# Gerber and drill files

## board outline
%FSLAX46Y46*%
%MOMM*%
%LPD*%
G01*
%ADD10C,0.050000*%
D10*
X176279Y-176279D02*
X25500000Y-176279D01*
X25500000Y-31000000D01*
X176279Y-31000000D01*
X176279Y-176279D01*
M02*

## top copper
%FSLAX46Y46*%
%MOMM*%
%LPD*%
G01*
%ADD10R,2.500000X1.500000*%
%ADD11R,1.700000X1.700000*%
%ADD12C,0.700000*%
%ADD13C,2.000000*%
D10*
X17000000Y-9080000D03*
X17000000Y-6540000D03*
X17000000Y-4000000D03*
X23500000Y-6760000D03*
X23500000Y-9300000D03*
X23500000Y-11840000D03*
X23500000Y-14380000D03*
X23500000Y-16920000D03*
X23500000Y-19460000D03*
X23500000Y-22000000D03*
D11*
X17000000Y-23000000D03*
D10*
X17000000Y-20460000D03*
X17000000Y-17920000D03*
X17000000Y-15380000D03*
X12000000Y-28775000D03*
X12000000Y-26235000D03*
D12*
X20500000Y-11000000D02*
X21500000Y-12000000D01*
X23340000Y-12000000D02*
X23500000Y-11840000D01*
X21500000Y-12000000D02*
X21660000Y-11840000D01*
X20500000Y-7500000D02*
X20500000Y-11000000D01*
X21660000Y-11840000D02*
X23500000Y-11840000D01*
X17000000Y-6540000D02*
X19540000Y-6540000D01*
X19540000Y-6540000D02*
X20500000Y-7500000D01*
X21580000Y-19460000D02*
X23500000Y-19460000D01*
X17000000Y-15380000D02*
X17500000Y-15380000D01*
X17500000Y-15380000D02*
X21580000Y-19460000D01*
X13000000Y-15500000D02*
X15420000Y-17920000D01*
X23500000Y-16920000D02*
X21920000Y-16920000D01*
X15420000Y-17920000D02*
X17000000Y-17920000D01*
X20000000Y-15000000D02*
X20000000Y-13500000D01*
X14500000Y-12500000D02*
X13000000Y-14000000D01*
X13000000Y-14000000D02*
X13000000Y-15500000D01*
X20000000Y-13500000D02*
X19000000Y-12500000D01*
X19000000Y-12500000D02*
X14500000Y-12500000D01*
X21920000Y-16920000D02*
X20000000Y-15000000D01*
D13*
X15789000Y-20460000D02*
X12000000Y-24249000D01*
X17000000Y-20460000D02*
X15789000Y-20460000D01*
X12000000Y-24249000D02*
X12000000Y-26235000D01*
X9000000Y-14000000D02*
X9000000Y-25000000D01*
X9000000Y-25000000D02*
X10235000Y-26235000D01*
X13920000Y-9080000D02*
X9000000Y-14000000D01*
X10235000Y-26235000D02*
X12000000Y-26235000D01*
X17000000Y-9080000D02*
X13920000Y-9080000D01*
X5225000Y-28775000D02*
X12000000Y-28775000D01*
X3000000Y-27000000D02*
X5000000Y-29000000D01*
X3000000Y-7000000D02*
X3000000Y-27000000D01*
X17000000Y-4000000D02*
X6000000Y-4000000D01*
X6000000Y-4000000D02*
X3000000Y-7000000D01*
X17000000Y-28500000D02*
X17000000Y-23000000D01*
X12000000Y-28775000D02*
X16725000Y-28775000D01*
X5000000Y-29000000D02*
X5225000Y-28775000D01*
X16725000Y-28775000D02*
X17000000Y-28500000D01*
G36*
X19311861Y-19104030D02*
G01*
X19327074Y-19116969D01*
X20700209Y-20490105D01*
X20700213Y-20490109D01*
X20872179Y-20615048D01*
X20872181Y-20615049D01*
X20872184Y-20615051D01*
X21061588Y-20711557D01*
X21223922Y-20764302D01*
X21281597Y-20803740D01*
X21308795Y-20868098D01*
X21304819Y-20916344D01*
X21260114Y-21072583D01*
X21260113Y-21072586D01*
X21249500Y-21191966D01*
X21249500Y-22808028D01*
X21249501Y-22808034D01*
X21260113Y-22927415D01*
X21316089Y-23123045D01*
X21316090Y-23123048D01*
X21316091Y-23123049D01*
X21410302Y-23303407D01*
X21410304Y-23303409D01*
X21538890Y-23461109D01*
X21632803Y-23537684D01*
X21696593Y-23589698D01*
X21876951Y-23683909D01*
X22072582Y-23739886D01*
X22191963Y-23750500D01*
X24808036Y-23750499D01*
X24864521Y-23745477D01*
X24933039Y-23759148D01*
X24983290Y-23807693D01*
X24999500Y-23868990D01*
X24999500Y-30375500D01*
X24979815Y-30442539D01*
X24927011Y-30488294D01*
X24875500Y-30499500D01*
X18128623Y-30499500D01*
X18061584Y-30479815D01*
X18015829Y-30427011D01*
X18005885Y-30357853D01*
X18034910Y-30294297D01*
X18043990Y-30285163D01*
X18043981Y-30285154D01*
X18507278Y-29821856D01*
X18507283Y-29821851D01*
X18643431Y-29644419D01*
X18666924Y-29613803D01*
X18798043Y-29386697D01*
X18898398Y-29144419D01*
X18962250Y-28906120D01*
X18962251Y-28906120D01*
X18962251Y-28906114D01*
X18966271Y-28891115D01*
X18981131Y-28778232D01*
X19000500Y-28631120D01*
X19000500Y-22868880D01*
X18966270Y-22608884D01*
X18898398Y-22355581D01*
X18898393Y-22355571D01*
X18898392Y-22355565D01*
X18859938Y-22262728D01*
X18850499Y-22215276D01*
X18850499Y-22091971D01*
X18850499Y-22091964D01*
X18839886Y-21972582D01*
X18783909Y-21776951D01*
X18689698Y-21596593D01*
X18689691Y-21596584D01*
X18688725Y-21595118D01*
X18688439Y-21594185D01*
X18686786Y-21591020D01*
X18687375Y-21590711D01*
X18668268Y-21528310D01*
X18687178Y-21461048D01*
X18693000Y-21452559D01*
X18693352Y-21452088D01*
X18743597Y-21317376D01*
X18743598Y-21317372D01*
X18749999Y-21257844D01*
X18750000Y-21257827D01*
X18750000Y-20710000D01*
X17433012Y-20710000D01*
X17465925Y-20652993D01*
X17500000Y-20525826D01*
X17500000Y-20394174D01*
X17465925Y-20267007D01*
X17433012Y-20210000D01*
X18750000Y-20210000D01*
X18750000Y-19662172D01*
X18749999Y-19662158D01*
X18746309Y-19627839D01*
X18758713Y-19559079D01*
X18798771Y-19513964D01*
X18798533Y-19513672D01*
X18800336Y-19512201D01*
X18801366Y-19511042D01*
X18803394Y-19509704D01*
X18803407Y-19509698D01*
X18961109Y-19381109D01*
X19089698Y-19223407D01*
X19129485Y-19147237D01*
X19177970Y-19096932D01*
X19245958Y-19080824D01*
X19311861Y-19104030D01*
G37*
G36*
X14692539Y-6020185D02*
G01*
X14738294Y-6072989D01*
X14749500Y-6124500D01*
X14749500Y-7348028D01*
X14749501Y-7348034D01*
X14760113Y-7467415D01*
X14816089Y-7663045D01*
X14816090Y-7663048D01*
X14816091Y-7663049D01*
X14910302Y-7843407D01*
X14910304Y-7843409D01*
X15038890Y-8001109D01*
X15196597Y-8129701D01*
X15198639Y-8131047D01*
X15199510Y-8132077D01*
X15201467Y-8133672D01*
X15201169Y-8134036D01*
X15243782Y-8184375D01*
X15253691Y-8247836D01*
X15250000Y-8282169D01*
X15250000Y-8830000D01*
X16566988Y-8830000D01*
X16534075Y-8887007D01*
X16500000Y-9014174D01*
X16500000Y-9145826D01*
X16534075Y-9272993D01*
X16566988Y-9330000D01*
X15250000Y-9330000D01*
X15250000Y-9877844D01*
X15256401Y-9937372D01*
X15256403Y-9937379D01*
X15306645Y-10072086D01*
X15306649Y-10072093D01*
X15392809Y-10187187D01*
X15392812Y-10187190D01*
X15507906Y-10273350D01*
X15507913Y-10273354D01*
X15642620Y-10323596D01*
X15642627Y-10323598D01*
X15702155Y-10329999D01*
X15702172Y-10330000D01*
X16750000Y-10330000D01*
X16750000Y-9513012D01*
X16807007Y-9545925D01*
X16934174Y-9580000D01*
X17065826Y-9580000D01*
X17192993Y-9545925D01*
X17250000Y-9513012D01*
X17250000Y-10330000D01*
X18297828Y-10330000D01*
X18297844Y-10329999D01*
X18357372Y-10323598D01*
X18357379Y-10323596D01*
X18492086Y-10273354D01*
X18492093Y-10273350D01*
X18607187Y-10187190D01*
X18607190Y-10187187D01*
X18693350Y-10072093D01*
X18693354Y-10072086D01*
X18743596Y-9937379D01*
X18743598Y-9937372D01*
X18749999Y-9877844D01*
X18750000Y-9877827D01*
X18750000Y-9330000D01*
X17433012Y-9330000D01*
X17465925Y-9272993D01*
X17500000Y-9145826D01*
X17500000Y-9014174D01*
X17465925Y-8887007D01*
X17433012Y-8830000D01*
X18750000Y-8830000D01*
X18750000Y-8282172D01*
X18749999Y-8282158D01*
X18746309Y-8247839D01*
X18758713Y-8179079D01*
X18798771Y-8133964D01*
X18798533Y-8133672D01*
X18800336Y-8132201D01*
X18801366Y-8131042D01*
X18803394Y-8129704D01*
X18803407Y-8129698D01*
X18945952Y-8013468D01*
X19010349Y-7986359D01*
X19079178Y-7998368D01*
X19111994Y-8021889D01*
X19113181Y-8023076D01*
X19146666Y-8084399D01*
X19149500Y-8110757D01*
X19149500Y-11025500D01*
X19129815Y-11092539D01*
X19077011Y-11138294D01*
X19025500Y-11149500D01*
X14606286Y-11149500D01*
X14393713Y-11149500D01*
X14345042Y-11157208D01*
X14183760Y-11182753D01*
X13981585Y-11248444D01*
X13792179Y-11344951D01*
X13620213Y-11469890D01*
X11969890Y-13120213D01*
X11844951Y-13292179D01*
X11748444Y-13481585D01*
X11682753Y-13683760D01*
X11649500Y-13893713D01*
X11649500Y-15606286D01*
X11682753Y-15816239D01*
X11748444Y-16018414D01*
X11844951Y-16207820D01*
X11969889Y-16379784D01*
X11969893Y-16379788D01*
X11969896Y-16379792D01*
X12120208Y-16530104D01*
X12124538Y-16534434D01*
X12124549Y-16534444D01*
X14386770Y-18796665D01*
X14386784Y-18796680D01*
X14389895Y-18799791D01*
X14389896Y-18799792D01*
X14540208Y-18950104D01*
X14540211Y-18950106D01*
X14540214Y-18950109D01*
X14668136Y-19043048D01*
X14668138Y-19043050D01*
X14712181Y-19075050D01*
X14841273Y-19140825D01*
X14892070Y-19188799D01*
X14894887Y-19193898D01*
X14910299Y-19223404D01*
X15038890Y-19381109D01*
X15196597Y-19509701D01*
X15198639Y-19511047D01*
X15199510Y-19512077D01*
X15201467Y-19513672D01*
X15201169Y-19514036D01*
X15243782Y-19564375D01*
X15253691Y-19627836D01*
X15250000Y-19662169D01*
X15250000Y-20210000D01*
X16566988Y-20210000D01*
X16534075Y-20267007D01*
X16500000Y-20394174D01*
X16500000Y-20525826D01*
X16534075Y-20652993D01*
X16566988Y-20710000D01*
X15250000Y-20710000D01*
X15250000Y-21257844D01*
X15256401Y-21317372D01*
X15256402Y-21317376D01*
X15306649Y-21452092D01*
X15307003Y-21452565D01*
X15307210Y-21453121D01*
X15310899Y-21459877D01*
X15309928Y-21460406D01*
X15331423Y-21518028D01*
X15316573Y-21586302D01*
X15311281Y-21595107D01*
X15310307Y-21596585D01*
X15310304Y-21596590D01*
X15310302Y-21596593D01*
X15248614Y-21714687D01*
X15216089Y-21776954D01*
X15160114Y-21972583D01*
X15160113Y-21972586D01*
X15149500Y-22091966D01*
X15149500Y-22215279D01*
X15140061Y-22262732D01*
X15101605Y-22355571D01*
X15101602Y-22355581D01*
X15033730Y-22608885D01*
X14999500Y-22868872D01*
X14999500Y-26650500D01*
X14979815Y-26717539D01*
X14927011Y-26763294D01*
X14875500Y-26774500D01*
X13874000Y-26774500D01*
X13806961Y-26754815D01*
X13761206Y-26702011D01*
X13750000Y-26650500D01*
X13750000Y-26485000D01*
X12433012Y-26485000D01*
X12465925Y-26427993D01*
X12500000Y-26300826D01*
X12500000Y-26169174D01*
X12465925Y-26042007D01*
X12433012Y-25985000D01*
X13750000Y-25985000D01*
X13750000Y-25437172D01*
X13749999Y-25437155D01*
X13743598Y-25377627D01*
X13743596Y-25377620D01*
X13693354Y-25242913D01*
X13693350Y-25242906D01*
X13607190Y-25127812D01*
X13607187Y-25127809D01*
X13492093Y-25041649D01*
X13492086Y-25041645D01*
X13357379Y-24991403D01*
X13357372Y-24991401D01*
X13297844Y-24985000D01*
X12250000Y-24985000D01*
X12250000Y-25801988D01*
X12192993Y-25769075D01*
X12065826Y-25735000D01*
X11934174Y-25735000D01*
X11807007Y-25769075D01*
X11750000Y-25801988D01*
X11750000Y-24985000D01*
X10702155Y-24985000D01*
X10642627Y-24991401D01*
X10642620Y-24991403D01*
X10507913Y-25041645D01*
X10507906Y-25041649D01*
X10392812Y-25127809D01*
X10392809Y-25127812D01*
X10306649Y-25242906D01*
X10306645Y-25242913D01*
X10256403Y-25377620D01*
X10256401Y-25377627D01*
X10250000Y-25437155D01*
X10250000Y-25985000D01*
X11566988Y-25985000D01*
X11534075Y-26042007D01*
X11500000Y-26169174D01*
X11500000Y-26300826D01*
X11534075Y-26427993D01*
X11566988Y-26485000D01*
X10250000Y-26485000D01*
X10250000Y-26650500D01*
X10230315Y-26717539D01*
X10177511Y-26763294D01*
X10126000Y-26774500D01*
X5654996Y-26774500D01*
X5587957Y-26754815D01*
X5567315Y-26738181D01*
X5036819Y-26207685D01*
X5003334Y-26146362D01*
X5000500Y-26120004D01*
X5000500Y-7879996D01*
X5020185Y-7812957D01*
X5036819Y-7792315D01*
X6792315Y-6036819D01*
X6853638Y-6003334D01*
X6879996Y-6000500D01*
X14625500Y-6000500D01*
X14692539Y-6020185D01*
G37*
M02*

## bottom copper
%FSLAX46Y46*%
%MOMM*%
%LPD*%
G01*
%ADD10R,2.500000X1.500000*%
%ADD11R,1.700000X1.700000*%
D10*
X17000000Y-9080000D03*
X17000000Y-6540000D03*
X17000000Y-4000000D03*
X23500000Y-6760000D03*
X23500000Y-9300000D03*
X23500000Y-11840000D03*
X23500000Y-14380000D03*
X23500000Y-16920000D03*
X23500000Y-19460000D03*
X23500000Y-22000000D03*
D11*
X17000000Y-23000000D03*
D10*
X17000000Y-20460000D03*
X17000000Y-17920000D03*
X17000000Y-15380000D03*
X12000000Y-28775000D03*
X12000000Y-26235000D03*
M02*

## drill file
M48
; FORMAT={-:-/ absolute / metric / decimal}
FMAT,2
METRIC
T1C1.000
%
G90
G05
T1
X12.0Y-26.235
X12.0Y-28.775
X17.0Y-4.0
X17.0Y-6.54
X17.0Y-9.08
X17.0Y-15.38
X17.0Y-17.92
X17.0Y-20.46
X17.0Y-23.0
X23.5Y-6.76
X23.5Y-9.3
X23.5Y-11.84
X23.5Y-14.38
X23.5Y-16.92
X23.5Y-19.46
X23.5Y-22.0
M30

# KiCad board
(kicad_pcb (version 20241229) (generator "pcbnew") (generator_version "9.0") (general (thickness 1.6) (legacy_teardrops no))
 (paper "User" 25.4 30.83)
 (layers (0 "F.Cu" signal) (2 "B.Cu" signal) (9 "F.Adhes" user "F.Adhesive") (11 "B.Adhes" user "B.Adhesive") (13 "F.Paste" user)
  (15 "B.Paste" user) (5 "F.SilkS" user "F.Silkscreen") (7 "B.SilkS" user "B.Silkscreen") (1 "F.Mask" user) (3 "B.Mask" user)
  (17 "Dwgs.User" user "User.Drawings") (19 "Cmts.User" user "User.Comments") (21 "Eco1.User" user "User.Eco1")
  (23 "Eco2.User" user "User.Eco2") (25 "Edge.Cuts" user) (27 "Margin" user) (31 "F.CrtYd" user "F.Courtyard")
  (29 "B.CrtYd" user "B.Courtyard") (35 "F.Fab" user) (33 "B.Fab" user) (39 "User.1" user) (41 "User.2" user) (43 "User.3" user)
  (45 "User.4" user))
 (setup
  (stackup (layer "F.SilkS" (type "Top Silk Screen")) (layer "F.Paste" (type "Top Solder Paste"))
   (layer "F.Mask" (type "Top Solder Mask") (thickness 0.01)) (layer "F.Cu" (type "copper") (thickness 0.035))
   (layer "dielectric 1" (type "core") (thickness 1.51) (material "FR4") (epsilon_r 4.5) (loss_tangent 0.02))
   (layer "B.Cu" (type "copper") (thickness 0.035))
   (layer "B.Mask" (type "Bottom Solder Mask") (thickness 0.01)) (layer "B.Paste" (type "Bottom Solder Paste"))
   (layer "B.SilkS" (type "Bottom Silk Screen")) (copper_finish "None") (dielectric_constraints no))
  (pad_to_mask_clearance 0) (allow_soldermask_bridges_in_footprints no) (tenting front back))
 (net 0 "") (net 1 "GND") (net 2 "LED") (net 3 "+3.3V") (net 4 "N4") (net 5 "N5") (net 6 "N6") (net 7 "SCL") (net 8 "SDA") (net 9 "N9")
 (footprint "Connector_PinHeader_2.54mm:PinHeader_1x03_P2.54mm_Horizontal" (layer "F.Cu") (at 17 9.08 180)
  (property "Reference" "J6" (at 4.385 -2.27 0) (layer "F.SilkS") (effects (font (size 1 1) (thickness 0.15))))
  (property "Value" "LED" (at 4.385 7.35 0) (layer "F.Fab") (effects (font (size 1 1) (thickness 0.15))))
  (pad "1" thru_hole rect (at 0 0 180) (size 2.5 1.5) (drill 1) (layers "*.Cu" "*.Mask") (remove_unused_layers no) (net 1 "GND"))
  (pad "2" thru_hole rect (at 0 2.54 180) (size 2.5 1.5) (drill 1) (layers "*.Cu" "*.Mask") (remove_unused_layers no) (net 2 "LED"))
  (pad "3" thru_hole rect (at 0 5.08 180) (size 2.5 1.5) (drill 1) (layers "*.Cu" "*.Mask") (remove_unused_layers no) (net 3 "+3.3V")))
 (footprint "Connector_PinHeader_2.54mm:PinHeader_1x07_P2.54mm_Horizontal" (layer "F.Cu") (at 23.5 6.76)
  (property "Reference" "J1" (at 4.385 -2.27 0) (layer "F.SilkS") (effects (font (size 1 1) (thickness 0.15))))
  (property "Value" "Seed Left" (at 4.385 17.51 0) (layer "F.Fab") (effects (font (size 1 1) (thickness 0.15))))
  (pad "1" thru_hole rect (at 0 0) (size 2.5 1.5) (drill 1) (layers "*.Cu" "*.Mask") (remove_unused_layers no) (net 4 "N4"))
  (pad "2" thru_hole rect (at 0 2.54) (size 2.5 1.5) (drill 1) (layers "*.Cu" "*.Mask") (remove_unused_layers no) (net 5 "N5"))
  (pad "3" thru_hole rect (at 0 5.08) (size 2.5 1.5) (drill 1) (layers "*.Cu" "*.Mask") (remove_unused_layers no) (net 2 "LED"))
  (pad "4" thru_hole rect (at 0 7.62) (size 2.5 1.5) (drill 1) (layers "*.Cu" "*.Mask") (remove_unused_layers no) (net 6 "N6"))
  (pad "5" thru_hole rect (at 0 10.16) (size 2.5 1.5) (drill 1) (layers "*.Cu" "*.Mask") (remove_unused_layers no) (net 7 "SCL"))
  (pad "6" thru_hole rect (at 0 12.7) (size 2.5 1.5) (drill 1) (layers "*.Cu" "*.Mask") (remove_unused_layers no) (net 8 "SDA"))
  (pad "7" thru_hole rect (at 0 15.24) (size 2.5 1.5) (drill 1) (layers "*.Cu" "*.Mask") (remove_unused_layers no) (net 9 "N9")))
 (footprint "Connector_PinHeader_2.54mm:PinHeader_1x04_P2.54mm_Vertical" (layer "F.Cu") (at 17 23 180)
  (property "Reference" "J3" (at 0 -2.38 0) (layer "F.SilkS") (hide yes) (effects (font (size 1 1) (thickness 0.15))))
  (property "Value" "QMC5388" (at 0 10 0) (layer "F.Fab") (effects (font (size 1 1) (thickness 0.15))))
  (pad "1" thru_hole rect (at 0 0 180) (size 1.7 1.7) (drill 1) (layers "*.Cu" "*.Mask") (remove_unused_layers no) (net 3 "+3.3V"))
  (pad "2" thru_hole rect (at 0 2.54 180) (size 2.5 1.5) (drill 1) (layers "*.Cu" "*.Mask") (remove_unused_layers no) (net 1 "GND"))
  (pad "3" thru_hole rect (at 0 5.08 180) (size 2.5 1.5) (drill 1) (layers "*.Cu" "*.Mask") (remove_unused_layers no) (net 7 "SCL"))
  (pad "4" thru_hole rect (at 0 7.62 180) (size 2.5 1.5) (drill 1) (layers "*.Cu" "*.Mask") (remove_unused_layers no) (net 8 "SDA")))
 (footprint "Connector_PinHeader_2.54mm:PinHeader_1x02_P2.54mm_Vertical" (layer "F.Cu") (at 12 28.775 180)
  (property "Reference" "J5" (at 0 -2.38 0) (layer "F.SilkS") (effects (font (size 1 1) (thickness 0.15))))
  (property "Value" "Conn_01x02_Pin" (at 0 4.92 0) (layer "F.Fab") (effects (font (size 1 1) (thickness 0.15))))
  (pad "1" thru_hole rect (at 0 0 180) (size 2.5 1.5) (drill 1) (layers "*.Cu" "*.Mask") (remove_unused_layers no) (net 3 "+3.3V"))
  (pad "2" thru_hole rect (at 0 2.54 180) (size 2.5 1.5) (drill 1) (layers "*.Cu" "*.Mask") (remove_unused_layers no) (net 1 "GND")))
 (gr_rect (start 0.176279 0.176279) (end 25.5 31) (stroke (width 0.05) (type default)) (fill no) (layer "Edge.Cuts"))
 (segment (start 20.5 11) (end 21.5 12) (width 0.7) (layer "F.Cu") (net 2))
 (segment (start 23.34 12) (end 23.5 11.84) (width 0.7) (layer "F.Cu") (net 2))
 (segment (start 21.5 12) (end 21.66 11.84) (width 0.7) (layer "F.Cu") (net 2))
 (segment (start 20.5 7.5) (end 20.5 11) (width 0.7) (layer "F.Cu") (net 2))
 (segment (start 21.66 11.84) (end 23.5 11.84) (width 0.7) (layer "F.Cu") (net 2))
 (segment (start 17 6.54) (end 19.54 6.54) (width 0.7) (layer "F.Cu") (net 2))
 (segment (start 19.54 6.54) (end 20.5 7.5) (width 0.7) (layer "F.Cu") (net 2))
 (segment (start 21.58 19.46) (end 23.5 19.46) (width 0.7) (layer "F.Cu") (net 8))
 (segment (start 17 15.38) (end 17.5 15.38) (width 0.7) (layer "F.Cu") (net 8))
 (segment (start 17.5 15.38) (end 21.58 19.46) (width 0.7) (layer "F.Cu") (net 8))
 (segment (start 13 15.5) (end 15.42 17.92) (width 0.7) (layer "F.Cu") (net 7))
 (segment (start 23.5 16.92) (end 21.92 16.92) (width 0.7) (layer "F.Cu") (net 7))
 (segment (start 15.42 17.92) (end 17 17.92) (width 0.7) (layer "F.Cu") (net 7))
 (segment (start 20 15) (end 20 13.5) (width 0.7) (layer "F.Cu") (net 7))
 (segment (start 14.5 12.5) (end 13 14) (width 0.7) (layer "F.Cu") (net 7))
 (segment (start 13 14) (end 13 15.5) (width 0.7) (layer "F.Cu") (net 7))
 (segment (start 20 13.5) (end 19 12.5) (width 0.7) (layer "F.Cu") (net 7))
 (segment (start 19 12.5) (end 14.5 12.5) (width 0.7) (layer "F.Cu") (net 7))
 (segment (start 21.92 16.92) (end 20 15) (width 0.7) (layer "F.Cu") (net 7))
 (segment (start 15.789 20.46) (end 12 24.249) (width 2) (layer "F.Cu") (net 1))
 (segment (start 17 20.46) (end 15.789 20.46) (width 2) (layer "F.Cu") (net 1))
 (segment (start 12 24.249) (end 12 26.235) (width 2) (layer "F.Cu") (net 1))
 (segment (start 9 14) (end 9 25) (width 2) (layer "F.Cu") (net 1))
 (segment (start 9 25) (end 10.235 26.235) (width 2) (layer "F.Cu") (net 1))
 (segment (start 13.92 9.08) (end 9 14) (width 2) (layer "F.Cu") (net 1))
 (segment (start 10.235 26.235) (end 12 26.235) (width 2) (layer "F.Cu") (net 1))
 (segment (start 17 9.08) (end 13.92 9.08) (width 2) (layer "F.Cu") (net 1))
 (segment (start 5.225 28.775) (end 12 28.775) (width 2) (layer "F.Cu") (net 3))
 (segment (start 3 27) (end 5 29) (width 2) (layer "F.Cu") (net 3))
 (segment (start 3 7) (end 3 27) (width 2) (layer "F.Cu") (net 3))
 (segment (start 17 4) (end 6 4) (width 2) (layer "F.Cu") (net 3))
 (segment (start 6 4) (end 3 7) (width 2) (layer "F.Cu") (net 3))
 (segment (start 17 28.5) (end 17 23) (width 2) (layer "F.Cu") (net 3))
 (segment (start 12 28.775) (end 16.725 28.775) (width 2) (layer "F.Cu") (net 3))
 (segment (start 5 29) (end 5.225 28.775) (width 2) (layer "F.Cu") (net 3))
 (segment (start 16.725 28.775) (end 17 28.5) (width 2) (layer "F.Cu") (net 3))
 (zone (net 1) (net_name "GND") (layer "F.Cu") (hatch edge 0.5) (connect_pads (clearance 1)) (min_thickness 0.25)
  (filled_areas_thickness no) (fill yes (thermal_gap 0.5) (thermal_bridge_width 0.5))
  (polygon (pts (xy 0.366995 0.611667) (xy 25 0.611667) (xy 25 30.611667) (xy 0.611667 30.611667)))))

